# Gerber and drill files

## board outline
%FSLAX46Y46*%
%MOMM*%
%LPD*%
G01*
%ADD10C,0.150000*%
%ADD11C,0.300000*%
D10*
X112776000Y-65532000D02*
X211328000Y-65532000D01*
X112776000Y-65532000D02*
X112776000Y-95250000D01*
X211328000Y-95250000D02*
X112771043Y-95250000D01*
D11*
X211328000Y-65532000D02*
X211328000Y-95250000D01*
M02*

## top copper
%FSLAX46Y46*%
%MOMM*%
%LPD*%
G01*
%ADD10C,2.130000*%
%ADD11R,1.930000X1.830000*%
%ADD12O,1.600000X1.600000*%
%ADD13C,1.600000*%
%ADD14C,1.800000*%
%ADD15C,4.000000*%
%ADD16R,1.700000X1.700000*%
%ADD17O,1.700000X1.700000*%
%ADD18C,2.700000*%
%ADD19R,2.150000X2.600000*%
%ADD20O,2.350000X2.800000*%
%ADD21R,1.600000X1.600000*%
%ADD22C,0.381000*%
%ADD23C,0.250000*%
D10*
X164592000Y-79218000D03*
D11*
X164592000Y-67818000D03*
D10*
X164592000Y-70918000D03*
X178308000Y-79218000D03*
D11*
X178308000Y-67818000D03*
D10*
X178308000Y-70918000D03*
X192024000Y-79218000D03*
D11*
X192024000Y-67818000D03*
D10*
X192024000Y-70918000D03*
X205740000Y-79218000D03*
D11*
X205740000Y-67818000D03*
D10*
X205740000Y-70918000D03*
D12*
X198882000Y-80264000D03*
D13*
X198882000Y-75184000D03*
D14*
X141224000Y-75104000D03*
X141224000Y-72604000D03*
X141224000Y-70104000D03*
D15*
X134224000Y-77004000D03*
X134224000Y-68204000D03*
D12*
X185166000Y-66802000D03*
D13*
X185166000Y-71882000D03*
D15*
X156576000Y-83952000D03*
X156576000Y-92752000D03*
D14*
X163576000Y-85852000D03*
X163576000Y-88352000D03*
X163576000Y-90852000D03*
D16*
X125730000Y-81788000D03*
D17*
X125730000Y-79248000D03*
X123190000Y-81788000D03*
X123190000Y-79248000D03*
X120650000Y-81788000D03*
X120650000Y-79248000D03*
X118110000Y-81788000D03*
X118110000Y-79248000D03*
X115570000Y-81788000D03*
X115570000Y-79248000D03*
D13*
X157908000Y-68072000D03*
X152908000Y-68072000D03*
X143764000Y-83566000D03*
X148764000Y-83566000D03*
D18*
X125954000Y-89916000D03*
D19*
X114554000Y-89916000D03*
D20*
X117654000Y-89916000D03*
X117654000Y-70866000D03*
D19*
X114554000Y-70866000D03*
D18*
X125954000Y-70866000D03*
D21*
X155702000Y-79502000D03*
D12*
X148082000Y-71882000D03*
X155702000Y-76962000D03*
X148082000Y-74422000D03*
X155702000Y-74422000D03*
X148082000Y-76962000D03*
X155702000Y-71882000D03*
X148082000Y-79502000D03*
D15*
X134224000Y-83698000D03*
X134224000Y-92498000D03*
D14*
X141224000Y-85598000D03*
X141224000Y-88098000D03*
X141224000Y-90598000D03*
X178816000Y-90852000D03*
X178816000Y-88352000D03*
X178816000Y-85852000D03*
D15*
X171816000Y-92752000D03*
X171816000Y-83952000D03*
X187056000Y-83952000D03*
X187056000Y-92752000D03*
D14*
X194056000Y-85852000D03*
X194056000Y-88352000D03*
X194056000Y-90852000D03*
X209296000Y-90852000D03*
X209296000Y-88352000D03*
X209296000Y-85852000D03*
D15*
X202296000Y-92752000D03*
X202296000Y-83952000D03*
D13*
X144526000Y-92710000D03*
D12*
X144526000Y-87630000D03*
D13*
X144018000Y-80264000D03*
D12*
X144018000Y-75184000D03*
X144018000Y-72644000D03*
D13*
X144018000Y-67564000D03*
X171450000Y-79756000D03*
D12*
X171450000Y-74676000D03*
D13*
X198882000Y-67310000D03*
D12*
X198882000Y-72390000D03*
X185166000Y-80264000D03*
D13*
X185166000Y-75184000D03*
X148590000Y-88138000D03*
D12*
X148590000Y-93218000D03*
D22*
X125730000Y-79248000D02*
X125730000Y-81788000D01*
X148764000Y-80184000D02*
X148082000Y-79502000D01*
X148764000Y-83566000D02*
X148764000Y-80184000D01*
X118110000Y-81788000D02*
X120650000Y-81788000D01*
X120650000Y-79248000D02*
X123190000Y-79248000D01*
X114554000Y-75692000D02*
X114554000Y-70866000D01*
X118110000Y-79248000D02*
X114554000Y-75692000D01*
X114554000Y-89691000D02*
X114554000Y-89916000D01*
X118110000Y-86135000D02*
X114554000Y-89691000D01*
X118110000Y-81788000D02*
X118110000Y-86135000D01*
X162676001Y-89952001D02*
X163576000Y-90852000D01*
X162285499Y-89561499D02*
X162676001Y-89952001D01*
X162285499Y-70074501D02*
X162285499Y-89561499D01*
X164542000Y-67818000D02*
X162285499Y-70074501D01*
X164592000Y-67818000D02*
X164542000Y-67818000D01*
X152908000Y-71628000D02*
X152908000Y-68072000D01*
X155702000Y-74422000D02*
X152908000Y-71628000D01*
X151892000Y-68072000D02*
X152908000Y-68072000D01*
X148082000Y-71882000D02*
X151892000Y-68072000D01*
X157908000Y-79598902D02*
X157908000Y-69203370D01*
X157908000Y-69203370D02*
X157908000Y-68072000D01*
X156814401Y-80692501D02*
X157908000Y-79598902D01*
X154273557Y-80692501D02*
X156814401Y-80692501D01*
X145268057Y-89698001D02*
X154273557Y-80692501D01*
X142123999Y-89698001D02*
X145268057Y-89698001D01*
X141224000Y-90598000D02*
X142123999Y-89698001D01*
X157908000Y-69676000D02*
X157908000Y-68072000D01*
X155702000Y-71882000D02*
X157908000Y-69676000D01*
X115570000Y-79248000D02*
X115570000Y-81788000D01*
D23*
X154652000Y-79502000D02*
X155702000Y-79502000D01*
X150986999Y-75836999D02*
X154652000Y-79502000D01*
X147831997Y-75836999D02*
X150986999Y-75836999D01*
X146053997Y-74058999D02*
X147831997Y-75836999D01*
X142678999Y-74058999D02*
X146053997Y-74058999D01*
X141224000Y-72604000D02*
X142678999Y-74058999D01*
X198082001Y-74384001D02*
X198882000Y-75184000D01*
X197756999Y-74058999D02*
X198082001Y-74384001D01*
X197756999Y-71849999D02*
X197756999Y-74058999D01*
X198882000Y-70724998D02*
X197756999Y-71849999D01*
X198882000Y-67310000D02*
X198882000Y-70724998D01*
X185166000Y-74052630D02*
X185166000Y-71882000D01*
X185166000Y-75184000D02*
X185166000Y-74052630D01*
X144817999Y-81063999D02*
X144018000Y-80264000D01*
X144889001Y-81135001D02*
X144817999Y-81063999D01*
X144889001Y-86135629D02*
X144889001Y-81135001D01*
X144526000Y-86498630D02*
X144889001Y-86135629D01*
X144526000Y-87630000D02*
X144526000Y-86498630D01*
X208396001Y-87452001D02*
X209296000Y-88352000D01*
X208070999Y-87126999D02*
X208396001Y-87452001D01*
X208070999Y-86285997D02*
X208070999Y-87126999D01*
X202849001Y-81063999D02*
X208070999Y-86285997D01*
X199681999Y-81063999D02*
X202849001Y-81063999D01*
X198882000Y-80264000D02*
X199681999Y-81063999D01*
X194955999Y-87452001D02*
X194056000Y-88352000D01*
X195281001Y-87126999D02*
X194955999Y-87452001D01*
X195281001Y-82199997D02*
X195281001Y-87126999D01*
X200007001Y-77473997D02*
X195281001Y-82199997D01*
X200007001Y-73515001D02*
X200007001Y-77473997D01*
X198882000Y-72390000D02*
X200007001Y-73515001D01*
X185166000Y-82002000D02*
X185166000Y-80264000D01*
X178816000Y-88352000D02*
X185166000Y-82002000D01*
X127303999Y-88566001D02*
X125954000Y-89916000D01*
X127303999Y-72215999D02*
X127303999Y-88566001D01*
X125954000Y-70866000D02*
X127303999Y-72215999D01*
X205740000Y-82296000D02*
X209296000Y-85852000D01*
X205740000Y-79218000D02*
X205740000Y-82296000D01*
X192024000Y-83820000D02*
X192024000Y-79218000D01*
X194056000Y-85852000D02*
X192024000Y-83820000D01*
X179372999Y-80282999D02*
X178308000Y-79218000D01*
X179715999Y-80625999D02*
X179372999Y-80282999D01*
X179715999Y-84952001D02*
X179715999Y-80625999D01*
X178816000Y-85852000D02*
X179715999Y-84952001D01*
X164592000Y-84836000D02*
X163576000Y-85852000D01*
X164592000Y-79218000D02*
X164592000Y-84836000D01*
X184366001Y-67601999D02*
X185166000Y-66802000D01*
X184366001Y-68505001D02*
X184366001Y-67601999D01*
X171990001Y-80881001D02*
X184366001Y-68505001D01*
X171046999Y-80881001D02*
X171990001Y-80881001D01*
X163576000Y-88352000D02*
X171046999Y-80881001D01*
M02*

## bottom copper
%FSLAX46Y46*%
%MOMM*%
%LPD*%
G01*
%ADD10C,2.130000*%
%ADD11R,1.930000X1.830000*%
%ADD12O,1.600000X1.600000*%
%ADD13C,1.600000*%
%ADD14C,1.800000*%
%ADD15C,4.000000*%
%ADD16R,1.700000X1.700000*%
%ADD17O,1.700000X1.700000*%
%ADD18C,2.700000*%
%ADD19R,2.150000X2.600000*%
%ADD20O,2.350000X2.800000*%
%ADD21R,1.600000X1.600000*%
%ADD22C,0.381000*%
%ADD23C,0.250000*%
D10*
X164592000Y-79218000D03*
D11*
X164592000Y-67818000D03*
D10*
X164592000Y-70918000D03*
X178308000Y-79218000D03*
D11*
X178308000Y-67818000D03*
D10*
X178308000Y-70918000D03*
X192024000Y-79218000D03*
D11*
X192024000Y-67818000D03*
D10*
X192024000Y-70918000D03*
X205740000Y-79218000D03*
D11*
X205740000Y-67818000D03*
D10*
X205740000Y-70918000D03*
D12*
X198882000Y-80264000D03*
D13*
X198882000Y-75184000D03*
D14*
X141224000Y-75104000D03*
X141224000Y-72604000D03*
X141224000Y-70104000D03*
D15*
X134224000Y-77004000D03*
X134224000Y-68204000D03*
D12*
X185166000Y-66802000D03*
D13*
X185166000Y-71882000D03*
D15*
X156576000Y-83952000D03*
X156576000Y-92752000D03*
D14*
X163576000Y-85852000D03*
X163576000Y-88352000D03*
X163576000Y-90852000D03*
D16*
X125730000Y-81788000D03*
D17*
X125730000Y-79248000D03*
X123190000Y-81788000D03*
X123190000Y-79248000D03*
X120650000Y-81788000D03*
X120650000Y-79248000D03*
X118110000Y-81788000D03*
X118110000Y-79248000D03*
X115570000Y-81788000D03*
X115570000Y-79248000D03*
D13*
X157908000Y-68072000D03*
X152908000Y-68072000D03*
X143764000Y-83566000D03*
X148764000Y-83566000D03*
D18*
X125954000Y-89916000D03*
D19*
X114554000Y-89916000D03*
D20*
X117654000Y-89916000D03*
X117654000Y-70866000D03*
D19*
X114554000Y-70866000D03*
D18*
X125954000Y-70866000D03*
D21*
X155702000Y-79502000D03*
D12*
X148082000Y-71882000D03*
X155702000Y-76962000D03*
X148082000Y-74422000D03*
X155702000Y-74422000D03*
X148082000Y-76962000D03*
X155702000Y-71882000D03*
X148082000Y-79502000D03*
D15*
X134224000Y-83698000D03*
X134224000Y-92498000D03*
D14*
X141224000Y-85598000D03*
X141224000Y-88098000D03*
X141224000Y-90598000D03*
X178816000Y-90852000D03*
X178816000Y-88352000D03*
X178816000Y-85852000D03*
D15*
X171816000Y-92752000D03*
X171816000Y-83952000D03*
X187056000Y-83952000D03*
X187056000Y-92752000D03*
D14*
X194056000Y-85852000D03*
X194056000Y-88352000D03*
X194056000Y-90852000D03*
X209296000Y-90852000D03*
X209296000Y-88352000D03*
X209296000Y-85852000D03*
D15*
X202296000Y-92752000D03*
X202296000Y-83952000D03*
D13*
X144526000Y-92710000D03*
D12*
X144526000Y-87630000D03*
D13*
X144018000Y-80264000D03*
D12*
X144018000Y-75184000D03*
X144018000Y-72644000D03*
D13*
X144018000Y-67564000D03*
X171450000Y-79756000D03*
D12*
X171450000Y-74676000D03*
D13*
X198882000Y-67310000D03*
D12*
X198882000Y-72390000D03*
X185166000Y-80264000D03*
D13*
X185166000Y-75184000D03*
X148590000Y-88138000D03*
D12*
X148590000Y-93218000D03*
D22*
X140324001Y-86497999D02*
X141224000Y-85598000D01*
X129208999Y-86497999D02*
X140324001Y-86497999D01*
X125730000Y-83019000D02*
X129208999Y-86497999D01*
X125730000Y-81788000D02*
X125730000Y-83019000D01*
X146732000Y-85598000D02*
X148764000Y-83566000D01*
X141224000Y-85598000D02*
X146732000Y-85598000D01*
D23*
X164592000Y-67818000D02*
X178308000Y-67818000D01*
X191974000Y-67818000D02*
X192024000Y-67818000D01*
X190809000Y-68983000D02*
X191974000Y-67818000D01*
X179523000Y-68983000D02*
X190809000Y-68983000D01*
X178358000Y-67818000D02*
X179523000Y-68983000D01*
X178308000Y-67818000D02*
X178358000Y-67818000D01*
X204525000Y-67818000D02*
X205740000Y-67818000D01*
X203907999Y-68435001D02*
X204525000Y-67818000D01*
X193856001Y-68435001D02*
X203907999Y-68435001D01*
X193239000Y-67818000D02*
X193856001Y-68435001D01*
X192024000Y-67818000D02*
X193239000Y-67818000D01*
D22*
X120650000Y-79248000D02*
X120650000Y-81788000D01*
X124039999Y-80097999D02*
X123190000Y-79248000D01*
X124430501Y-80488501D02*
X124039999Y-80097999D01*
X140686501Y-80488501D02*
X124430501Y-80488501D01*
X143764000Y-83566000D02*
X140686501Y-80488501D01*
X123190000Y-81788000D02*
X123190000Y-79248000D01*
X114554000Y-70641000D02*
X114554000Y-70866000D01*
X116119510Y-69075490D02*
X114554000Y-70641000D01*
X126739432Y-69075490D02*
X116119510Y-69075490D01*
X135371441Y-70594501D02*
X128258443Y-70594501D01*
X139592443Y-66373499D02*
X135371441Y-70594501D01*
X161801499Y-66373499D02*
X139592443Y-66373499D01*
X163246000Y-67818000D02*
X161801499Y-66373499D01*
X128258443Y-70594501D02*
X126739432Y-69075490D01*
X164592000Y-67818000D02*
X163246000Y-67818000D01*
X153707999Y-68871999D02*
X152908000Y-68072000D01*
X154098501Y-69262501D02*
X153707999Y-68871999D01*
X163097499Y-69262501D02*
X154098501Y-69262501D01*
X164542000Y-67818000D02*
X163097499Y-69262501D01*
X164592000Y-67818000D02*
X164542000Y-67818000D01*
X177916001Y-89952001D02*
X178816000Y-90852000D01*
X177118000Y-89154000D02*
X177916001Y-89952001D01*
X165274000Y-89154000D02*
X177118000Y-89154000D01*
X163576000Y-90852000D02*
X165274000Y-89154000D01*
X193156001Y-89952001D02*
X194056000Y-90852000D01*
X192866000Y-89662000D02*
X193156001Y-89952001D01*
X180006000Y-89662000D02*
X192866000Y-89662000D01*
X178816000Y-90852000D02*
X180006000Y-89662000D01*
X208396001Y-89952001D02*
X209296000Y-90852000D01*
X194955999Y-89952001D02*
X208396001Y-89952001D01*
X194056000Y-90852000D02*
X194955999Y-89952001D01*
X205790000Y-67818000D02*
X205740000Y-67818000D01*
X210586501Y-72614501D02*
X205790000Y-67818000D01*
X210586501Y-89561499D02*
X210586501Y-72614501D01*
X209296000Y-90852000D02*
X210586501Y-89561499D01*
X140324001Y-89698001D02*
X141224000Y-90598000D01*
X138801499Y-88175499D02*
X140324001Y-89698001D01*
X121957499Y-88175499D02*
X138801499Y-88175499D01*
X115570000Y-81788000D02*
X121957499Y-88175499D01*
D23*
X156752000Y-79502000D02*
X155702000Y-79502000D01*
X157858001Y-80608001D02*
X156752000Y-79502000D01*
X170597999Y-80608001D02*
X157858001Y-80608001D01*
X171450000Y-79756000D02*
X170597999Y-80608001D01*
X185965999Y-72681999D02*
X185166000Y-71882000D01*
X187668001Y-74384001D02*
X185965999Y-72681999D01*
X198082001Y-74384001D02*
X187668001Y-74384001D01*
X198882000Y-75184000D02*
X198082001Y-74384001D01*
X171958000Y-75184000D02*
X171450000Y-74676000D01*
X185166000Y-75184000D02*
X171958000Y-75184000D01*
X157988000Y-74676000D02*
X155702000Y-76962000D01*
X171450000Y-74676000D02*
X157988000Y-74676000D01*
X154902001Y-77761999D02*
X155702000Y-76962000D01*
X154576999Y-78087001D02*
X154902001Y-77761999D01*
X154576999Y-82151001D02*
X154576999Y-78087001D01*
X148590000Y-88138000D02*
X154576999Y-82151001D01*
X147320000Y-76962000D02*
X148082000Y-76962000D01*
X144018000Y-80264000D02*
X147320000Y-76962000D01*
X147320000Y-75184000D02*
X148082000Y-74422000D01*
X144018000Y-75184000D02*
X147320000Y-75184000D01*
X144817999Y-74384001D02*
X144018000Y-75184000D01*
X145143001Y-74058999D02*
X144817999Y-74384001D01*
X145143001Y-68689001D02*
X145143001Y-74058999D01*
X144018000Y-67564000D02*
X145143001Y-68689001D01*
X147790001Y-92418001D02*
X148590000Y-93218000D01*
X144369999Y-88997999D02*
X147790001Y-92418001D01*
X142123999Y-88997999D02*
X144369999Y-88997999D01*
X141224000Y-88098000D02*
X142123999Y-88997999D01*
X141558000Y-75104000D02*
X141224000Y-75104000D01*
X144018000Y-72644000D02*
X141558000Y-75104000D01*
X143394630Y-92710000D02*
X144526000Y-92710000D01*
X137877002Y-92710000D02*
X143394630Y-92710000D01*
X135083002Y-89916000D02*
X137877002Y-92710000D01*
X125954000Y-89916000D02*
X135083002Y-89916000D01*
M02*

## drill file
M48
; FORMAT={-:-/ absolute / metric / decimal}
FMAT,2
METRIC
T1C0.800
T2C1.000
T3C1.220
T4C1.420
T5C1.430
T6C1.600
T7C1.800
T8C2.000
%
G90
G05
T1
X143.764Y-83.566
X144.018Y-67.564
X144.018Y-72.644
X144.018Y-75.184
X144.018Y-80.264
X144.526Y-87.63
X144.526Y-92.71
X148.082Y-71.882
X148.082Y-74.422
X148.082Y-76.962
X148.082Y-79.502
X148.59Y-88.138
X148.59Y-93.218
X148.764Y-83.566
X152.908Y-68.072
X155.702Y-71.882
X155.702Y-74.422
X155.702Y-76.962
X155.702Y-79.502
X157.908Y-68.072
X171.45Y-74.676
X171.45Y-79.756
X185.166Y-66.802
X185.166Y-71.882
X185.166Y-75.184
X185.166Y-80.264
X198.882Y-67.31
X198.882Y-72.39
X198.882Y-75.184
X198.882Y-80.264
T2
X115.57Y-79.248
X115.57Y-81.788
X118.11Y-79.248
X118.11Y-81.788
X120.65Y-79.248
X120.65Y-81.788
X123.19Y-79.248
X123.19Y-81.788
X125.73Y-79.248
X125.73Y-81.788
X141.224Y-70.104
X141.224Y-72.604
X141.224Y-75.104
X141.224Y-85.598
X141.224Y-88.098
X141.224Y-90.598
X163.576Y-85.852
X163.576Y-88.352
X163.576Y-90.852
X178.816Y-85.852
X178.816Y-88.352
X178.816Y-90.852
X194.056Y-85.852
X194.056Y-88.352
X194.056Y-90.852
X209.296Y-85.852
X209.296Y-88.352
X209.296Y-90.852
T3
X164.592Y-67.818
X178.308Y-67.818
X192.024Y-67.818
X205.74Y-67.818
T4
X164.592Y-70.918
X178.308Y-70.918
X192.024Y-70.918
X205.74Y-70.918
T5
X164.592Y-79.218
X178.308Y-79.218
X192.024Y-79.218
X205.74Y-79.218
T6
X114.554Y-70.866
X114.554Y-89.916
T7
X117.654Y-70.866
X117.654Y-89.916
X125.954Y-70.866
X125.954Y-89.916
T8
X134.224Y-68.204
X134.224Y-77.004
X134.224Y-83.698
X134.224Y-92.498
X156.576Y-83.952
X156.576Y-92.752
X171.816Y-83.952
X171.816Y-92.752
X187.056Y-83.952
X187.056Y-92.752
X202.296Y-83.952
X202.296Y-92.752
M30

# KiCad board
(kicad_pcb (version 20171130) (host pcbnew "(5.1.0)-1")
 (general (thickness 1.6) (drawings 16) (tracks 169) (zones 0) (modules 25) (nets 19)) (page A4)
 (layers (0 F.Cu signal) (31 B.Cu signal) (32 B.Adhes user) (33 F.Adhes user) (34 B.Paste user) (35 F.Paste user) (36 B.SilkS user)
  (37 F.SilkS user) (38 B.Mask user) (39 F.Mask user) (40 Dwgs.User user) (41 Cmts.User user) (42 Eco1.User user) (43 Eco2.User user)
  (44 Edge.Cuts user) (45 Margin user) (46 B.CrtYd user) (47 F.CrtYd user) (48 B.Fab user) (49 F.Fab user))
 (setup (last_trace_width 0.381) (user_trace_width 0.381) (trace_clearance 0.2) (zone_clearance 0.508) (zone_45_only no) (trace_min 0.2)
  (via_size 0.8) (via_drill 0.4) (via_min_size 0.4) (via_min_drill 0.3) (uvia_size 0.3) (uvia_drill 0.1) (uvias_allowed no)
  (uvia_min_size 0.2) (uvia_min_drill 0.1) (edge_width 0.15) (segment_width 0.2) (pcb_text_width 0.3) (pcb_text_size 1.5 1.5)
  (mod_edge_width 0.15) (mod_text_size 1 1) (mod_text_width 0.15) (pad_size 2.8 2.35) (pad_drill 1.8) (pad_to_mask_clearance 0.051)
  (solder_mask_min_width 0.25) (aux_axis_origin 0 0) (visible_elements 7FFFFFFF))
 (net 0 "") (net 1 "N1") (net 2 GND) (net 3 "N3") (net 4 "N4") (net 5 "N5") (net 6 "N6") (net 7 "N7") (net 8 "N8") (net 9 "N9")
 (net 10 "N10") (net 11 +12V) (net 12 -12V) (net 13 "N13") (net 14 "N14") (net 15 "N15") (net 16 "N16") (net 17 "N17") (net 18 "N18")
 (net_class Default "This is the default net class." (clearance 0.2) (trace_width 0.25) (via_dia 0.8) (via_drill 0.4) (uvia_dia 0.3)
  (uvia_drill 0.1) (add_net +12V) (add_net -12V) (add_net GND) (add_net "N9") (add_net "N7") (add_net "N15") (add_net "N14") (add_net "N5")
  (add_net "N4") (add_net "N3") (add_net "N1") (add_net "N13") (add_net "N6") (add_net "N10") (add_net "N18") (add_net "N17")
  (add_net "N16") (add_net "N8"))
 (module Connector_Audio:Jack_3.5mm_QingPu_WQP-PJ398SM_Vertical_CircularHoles (layer F.Cu) (at 164.592 67.818)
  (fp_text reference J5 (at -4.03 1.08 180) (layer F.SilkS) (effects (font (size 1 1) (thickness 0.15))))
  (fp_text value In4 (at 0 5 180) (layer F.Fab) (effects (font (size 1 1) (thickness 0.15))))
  (pad T thru_hole circle (at 0 11.4 180) (size 2.13 2.13) (drill 1.43) (layers *.Cu *.Mask) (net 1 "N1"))
  (pad S thru_hole rect (at 0 0 180) (size 1.93 1.83) (drill 1.22) (layers *.Cu *.Mask) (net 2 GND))
  (pad TN thru_hole circle (at 0 3.1 180) (size 2.13 2.13) (drill 1.42) (layers *.Cu *.Mask)))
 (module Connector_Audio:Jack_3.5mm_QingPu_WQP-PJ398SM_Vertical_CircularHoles (layer F.Cu) (at 178.308 67.818)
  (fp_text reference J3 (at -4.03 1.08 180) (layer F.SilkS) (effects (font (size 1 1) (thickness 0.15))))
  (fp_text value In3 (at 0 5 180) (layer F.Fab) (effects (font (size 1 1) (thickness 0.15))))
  (pad T thru_hole circle (at 0 11.4 180) (size 2.13 2.13) (drill 1.43) (layers *.Cu *.Mask) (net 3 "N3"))
  (pad S thru_hole rect (at 0 0 180) (size 1.93 1.83) (drill 1.22) (layers *.Cu *.Mask) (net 2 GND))
  (pad TN thru_hole circle (at 0 3.1 180) (size 2.13 2.13) (drill 1.42) (layers *.Cu *.Mask)))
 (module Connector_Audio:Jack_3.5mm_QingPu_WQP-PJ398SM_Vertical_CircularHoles (layer F.Cu) (at 192.024 67.818)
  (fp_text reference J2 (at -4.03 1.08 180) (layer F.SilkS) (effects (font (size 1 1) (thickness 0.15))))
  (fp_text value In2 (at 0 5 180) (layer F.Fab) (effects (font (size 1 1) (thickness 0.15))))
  (pad T thru_hole circle (at 0 11.4 180) (size 2.13 2.13) (drill 1.43) (layers *.Cu *.Mask) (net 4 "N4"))
  (pad S thru_hole rect (at 0 0 180) (size 1.93 1.83) (drill 1.22) (layers *.Cu *.Mask) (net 2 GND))
  (pad TN thru_hole circle (at 0 3.1 180) (size 2.13 2.13) (drill 1.42) (layers *.Cu *.Mask)))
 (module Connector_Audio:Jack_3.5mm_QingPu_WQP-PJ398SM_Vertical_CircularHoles (layer F.Cu) (at 205.74 67.818)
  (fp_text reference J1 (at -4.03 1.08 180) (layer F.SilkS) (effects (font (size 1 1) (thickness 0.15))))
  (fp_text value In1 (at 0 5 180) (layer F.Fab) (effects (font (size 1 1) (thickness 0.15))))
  (pad T thru_hole circle (at 0 11.4 180) (size 2.13 2.13) (drill 1.43) (layers *.Cu *.Mask) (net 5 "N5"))
  (pad S thru_hole rect (at 0 0 180) (size 1.93 1.83) (drill 1.22) (layers *.Cu *.Mask) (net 2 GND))
  (pad TN thru_hole circle (at 0 3.1 180) (size 2.13 2.13) (drill 1.42) (layers *.Cu *.Mask)))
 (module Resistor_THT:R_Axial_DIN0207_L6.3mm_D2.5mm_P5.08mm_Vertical (layer F.Cu) (at 198.882 75.184 270)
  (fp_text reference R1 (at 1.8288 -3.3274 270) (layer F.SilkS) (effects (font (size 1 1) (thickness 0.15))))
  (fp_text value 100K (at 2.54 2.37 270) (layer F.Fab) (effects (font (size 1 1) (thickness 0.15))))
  (pad 2 thru_hole oval (at 5.08 0 270) (size 1.6 1.6) (drill 0.8) (layers *.Cu *.Mask) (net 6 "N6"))
  (pad 1 thru_hole circle (at 0 0 270) (size 1.6 1.6) (drill 0.8) (layers *.Cu *.Mask) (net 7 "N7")))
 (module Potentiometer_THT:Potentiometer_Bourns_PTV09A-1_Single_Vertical (layer F.Cu) (at 141.224 70.104 180)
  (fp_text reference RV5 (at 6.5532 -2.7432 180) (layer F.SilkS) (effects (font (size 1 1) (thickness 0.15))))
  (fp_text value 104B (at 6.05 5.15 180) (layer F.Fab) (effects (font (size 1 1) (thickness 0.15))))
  (pad 3 thru_hole circle (at 0 -5 180) (size 1.8 1.8) (drill 1) (layers *.Cu *.Mask) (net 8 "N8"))
  (pad 2 thru_hole circle (at 0 -2.5 180) (size 1.8 1.8) (drill 1) (layers *.Cu *.Mask) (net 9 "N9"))
  (pad 1 thru_hole circle (at 0 0 180) (size 1.8 1.8) (drill 1) (layers *.Cu *.Mask))
  (pad "" np_thru_hole circle (at 7 -6.9 180) (size 4 4) (drill 2) (layers *.Cu *.Mask))
  (pad "" np_thru_hole circle (at 7 1.9 180) (size 4 4) (drill 2) (layers *.Cu *.Mask)))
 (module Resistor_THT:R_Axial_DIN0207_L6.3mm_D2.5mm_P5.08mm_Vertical (layer F.Cu) (at 185.166 71.882 90)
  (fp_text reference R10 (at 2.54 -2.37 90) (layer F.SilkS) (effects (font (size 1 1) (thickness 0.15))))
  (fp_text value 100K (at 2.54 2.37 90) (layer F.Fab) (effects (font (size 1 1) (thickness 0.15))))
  (pad 2 thru_hole oval (at 5.08 0 90) (size 1.6 1.6) (drill 0.8) (layers *.Cu *.Mask) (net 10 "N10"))
  (pad 1 thru_hole circle (at 0 0 90) (size 1.6 1.6) (drill 0.8) (layers *.Cu *.Mask) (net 7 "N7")))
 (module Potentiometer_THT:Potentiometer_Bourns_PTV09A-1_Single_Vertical (layer F.Cu) (at 163.576 85.852 180)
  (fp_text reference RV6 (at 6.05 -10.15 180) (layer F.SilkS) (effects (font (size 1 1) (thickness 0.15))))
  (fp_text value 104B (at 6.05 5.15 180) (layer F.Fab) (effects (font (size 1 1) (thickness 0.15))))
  (pad "" np_thru_hole circle (at 7 1.9 180) (size 4 4) (drill 2) (layers *.Cu *.Mask))
  (pad "" np_thru_hole circle (at 7 -6.9 180) (size 4 4) (drill 2) (layers *.Cu *.Mask))
  (pad 1 thru_hole circle (at 0 0 180) (size 1.8 1.8) (drill 1) (layers *.Cu *.Mask) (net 1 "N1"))
  (pad 2 thru_hole circle (at 0 -2.5 180) (size 1.8 1.8) (drill 1) (layers *.Cu *.Mask) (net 10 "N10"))
  (pad 3 thru_hole circle (at 0 -5 180) (size 1.8 1.8) (drill 1) (layers *.Cu *.Mask) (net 2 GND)))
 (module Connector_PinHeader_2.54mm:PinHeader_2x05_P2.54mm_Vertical (layer B.Cu) (at 125.73 81.788 90)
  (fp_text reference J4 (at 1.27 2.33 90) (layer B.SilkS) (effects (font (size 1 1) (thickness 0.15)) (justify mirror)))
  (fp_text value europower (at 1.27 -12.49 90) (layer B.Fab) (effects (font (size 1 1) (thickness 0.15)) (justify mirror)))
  (pad 1 thru_hole rect (at 0 0 90) (size 1.7 1.7) (drill 1) (layers *.Cu *.Mask) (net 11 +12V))
  (pad 2 thru_hole oval (at 2.54 0 90) (size 1.7 1.7) (drill 1) (layers *.Cu *.Mask) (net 11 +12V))
  (pad 3 thru_hole oval (at 0 -2.54 90) (size 1.7 1.7) (drill 1) (layers *.Cu *.Mask) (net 2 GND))
  (pad 4 thru_hole oval (at 2.54 -2.54 90) (size 1.7 1.7) (drill 1) (layers *.Cu *.Mask) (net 2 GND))
  (pad 5 thru_hole oval (at 0 -5.08 90) (size 1.7 1.7) (drill 1) (layers *.Cu *.Mask) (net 2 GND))
  (pad 6 thru_hole oval (at 2.54 -5.08 90) (size 1.7 1.7) (drill 1) (layers *.Cu *.Mask) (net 2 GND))
  (pad 7 thru_hole oval (at 0 -7.62 90) (size 1.7 1.7) (drill 1) (layers *.Cu *.Mask) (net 2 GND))
  (pad 8 thru_hole oval (at 2.54 -7.62 90) (size 1.7 1.7) (drill 1) (layers *.Cu *.Mask) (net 2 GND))
  (pad 9 thru_hole oval (at 0 -10.16 90) (size 1.7 1.7) (drill 1) (layers *.Cu *.Mask) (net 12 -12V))
  (pad 10 thru_hole oval (at 2.54 -10.16 90) (size 1.7 1.7) (drill 1) (layers *.Cu *.Mask) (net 12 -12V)))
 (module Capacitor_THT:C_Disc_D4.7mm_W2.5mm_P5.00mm (layer F.Cu) (at 152.908 68.072)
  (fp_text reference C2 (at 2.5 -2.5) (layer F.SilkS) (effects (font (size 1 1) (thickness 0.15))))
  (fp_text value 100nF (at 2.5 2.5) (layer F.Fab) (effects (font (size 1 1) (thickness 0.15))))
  (pad 2 thru_hole circle (at 5 0) (size 1.6 1.6) (drill 0.8) (layers *.Cu *.Mask) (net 12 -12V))
  (pad 1 thru_hole circle (at 0 0) (size 1.6 1.6) (drill 0.8) (layers *.Cu *.Mask) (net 2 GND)))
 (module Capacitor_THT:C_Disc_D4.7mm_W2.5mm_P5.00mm (layer F.Cu) (at 143.764 83.566)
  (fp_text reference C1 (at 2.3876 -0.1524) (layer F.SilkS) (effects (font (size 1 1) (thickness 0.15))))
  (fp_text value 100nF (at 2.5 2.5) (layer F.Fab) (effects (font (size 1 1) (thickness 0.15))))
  (pad 1 thru_hole circle (at 0 0) (size 1.6 1.6) (drill 0.8) (layers *.Cu *.Mask) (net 2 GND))
  (pad 2 thru_hole circle (at 5 0) (size 1.6 1.6) (drill 0.8) (layers *.Cu *.Mask) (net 11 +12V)))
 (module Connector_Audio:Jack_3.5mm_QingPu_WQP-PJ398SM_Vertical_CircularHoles (layer F.Cu) (at 114.554 89.916 90)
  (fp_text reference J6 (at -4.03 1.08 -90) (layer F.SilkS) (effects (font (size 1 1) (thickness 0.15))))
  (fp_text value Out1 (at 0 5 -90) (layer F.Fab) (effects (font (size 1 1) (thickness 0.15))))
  (pad T thru_hole circle (at 0 11.4 270) (size 2.7 2.7) (drill 1.8) (layers *.Cu *.Mask) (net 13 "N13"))
  (pad S thru_hole rect (at 0 0 270) (size 2.6 2.15) (drill 1.6) (layers *.Cu *.Mask) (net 2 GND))
  (pad TN thru_hole oval (at 0 3.1 270) (size 2.8 2.35) (drill 1.8) (layers *.Cu *.Mask)))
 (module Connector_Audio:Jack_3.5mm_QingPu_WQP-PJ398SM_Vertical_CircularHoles (layer F.Cu) (at 114.554 70.866 90)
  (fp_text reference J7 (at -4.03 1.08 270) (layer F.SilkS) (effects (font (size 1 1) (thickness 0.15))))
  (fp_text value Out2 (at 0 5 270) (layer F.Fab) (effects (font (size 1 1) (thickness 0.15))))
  (pad TN thru_hole oval (at 0 3.1 270) (size 2.8 2.35) (drill 1.8) (layers *.Cu *.Mask))
  (pad S thru_hole rect (at 0 0 270) (size 2.6 2.15) (drill 1.6) (layers *.Cu *.Mask) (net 2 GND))
  (pad T thru_hole circle (at 0 11.4 270) (size 2.7 2.7) (drill 1.8) (layers *.Cu *.Mask) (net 13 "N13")))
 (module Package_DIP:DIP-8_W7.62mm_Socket (layer F.Cu) (at 155.702 79.502 180)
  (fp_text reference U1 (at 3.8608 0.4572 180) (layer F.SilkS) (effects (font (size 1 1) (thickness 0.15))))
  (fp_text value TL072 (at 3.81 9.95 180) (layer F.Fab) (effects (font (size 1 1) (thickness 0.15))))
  (pad 1 thru_hole rect (at 0 0 180) (size 1.6 1.6) (drill 0.8) (layers *.Cu *.Mask) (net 9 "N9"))
  (pad 5 thru_hole oval (at 7.62 7.62 180) (size 1.6 1.6) (drill 0.8) (layers *.Cu *.Mask) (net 2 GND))
  (pad 2 thru_hole oval (at 0 2.54 180) (size 1.6 1.6) (drill 0.8) (layers *.Cu *.Mask) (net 7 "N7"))
  (pad 6 thru_hole oval (at 7.62 5.08 180) (size 1.6 1.6) (drill 0.8) (layers *.Cu *.Mask) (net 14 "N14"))
  (pad 3 thru_hole oval (at 0 5.08 180) (size 1.6 1.6) (drill 0.8) (layers *.Cu *.Mask) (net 2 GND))
  (pad 7 thru_hole oval (at 7.62 2.54 180) (size 1.6 1.6) (drill 0.8) (layers *.Cu *.Mask) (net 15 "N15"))
  (pad 4 thru_hole oval (at 0 7.62 180) (size 1.6 1.6) (drill 0.8) (layers *.Cu *.Mask) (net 12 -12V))
  (pad 8 thru_hole oval (at 7.62 0 180) (size 1.6 1.6) (drill 0.8) (layers *.Cu *.Mask) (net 11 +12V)))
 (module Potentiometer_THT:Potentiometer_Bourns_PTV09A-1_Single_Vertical (layer F.Cu) (at 141.224 85.598 180)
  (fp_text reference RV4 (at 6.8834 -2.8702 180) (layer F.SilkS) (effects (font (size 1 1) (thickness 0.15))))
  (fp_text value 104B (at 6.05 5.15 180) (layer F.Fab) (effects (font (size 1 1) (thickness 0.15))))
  (pad "" np_thru_hole circle (at 7 1.9 180) (size 4 4) (drill 2) (layers *.Cu *.Mask))
  (pad "" np_thru_hole circle (at 7 -6.9 180) (size 4 4) (drill 2) (layers *.Cu *.Mask))
  (pad 1 thru_hole circle (at 0 0 180) (size 1.8 1.8) (drill 1) (layers *.Cu *.Mask) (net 11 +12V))
  (pad 2 thru_hole circle (at 0 -2.5 180) (size 1.8 1.8) (drill 1) (layers *.Cu *.Mask) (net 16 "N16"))
  (pad 3 thru_hole circle (at 0 -5 180) (size 1.8 1.8) (drill 1) (layers *.Cu *.Mask) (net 12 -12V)))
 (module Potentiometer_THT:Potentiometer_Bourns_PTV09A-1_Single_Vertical (layer F.Cu) (at 178.816 85.852 180)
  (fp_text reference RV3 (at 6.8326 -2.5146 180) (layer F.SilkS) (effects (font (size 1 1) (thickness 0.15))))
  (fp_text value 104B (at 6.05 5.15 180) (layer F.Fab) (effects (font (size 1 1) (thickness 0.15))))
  (pad 3 thru_hole circle (at 0 -5 180) (size 1.8 1.8) (drill 1) (layers *.Cu *.Mask) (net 2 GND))
  (pad 2 thru_hole circle (at 0 -2.5 180) (size 1.8 1.8) (drill 1) (layers *.Cu *.Mask) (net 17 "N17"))
  (pad 1 thru_hole circle (at 0 0 180) (size 1.8 1.8) (drill 1) (layers *.Cu *.Mask) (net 3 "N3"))
  (pad "" np_thru_hole circle (at 7 -6.9 180) (size 4 4) (drill 2) (layers *.Cu *.Mask))
  (pad "" np_thru_hole circle (at 7 1.9 180) (size 4 4) (drill 2) (layers *.Cu *.Mask)))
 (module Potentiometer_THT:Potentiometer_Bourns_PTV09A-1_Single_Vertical (layer F.Cu) (at 194.056 85.852 180)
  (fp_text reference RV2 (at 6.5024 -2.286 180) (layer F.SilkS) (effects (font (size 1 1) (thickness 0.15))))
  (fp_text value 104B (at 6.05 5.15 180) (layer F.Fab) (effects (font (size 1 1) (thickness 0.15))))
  (pad "" np_thru_hole circle (at 7 1.9 180) (size 4 4) (drill 2) (layers *.Cu *.Mask))
  (pad "" np_thru_hole circle (at 7 -6.9 180) (size 4 4) (drill 2) (layers *.Cu *.Mask))
  (pad 1 thru_hole circle (at 0 0 180) (size 1.8 1.8) (drill 1) (layers *.Cu *.Mask) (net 4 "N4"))
  (pad 2 thru_hole circle (at 0 -2.5 180) (size 1.8 1.8) (drill 1) (layers *.Cu *.Mask) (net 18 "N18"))
  (pad 3 thru_hole circle (at 0 -5 180) (size 1.8 1.8) (drill 1) (layers *.Cu *.Mask) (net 2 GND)))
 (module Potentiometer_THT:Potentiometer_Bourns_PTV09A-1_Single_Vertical (layer F.Cu) (at 209.296 85.852 180)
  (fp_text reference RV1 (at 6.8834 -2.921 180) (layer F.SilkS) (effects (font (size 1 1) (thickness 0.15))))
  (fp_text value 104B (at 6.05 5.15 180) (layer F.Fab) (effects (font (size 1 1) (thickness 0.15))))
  (pad 3 thru_hole circle (at 0 -5 180) (size 1.8 1.8) (drill 1) (layers *.Cu *.Mask) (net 2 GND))
  (pad 2 thru_hole circle (at 0 -2.5 180) (size 1.8 1.8) (drill 1) (layers *.Cu *.Mask) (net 6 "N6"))
  (pad 1 thru_hole circle (at 0 0 180) (size 1.8 1.8) (drill 1) (layers *.Cu *.Mask) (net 5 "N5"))
  (pad "" np_thru_hole circle (at 7 -6.9 180) (size 4 4) (drill 2) (layers *.Cu *.Mask))
  (pad "" np_thru_hole circle (at 7 1.9 180) (size 4 4) (drill 2) (layers *.Cu *.Mask)))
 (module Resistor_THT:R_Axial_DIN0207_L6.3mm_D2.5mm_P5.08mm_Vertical (layer F.Cu) (at 144.526 92.71 90)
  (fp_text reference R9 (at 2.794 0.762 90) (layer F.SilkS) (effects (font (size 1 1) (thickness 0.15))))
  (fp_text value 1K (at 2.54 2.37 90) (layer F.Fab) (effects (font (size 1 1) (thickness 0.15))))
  (pad 1 thru_hole circle (at 0 0 90) (size 1.6 1.6) (drill 0.8) (layers *.Cu *.Mask) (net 13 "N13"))
  (pad 2 thru_hole oval (at 5.08 0 90) (size 1.6 1.6) (drill 0.8) (layers *.Cu *.Mask) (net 15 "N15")))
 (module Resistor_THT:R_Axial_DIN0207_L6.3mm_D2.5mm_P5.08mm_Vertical (layer F.Cu) (at 144.018 80.264 90)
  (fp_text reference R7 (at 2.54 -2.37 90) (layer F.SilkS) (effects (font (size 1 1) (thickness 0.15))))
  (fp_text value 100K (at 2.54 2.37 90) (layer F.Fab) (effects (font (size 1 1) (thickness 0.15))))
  (pad 1 thru_hole circle (at 0 0 90) (size 1.6 1.6) (drill 0.8) (layers *.Cu *.Mask) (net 15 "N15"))
  (pad 2 thru_hole oval (at 5.08 0 90) (size 1.6 1.6) (drill 0.8) (layers *.Cu *.Mask) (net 14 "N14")))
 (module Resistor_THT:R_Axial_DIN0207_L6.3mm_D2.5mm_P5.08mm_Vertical (layer F.Cu) (at 144.018 67.564 270)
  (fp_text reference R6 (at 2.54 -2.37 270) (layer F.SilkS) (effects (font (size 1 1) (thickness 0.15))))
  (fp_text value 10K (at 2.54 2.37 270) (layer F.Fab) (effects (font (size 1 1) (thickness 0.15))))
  (pad 2 thru_hole oval (at 5.08 0 270) (size 1.6 1.6) (drill 0.8) (layers *.Cu *.Mask) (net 8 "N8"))
  (pad 1 thru_hole circle (at 0 0 270) (size 1.6 1.6) (drill 0.8) (layers *.Cu *.Mask) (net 14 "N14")))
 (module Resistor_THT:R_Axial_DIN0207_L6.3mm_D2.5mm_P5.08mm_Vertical (layer F.Cu) (at 171.45 79.756 90)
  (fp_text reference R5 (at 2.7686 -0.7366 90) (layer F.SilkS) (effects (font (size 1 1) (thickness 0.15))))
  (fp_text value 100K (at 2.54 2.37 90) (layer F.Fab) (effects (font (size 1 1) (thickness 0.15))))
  (pad 1 thru_hole circle (at 0 0 90) (size 1.6 1.6) (drill 0.8) (layers *.Cu *.Mask) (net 9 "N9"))
  (pad 2 thru_hole oval (at 5.08 0 90) (size 1.6 1.6) (drill 0.8) (layers *.Cu *.Mask) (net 7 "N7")))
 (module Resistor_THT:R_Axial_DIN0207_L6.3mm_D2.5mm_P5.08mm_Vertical (layer F.Cu) (at 198.882 67.31 270)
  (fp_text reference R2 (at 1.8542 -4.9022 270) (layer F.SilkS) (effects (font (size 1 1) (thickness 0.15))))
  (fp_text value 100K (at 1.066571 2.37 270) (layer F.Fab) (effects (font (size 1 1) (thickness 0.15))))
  (pad 1 thru_hole circle (at 0 0 270) (size 1.6 1.6) (drill 0.8) (layers *.Cu *.Mask) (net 7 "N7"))
  (pad 2 thru_hole oval (at 5.08 0 270) (size 1.6 1.6) (drill 0.8) (layers *.Cu *.Mask) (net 18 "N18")))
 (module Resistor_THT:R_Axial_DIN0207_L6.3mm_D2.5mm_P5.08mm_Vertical (layer F.Cu) (at 185.166 75.184 270)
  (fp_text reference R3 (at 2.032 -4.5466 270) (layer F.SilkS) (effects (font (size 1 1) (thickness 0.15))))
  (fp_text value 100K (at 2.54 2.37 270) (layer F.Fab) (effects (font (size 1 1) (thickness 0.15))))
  (pad 2 thru_hole oval (at 5.08 0 270) (size 1.6 1.6) (drill 0.8) (layers *.Cu *.Mask) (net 17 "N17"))
  (pad 1 thru_hole circle (at 0 0 270) (size 1.6 1.6) (drill 0.8) (layers *.Cu *.Mask) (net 7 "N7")))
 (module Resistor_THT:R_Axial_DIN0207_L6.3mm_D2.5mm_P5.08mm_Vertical (layer F.Cu) (at 148.59 88.138 270)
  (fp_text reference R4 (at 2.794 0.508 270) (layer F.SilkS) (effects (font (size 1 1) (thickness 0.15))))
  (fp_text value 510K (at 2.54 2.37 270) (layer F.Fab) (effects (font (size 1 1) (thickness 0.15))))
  (pad 1 thru_hole circle (at 0 0 270) (size 1.6 1.6) (drill 0.8) (layers *.Cu *.Mask) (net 7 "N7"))
  (pad 2 thru_hole oval (at 5.08 0 270) (size 1.6 1.6) (drill 0.8) (layers *.Cu *.Mask) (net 16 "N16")))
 (gr_line (start 112.776 65.532) (end 211.328 65.532) (layer Edge.Cuts) (width 0.15))
 (gr_line (start 112.776 65.532) (end 112.776 95.25) (layer Edge.Cuts) (width 0.15))
 (gr_line (start 211.328 95.25) (end 112.771043 95.25) (layer Edge.Cuts) (width 0.15))
 (gr_line (start 211.328 65.532) (end 211.328 95.25) (layer Edge.Cuts) (width 0.3))
 (segment (start 140.324001 86.497999) (end 141.224 85.598) (width 0.381) (layer B.Cu) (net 11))
 (segment (start 129.208999 86.497999) (end 140.324001 86.497999) (width 0.381) (layer B.Cu) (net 11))
 (segment (start 125.73 83.019) (end 129.208999 86.497999) (width 0.381) (layer B.Cu) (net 11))
 (segment (start 125.73 81.788) (end 125.73 83.019) (width 0.381) (layer B.Cu) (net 11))
 (segment (start 146.732 85.598) (end 148.764 83.566) (width 0.381) (layer B.Cu) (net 11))
 (segment (start 141.224 85.598) (end 146.732 85.598) (width 0.381) (layer B.Cu) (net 11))
 (segment (start 125.73 79.248) (end 125.73 81.788) (width 0.381) (layer F.Cu) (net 11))
 (segment (start 148.764 80.184) (end 148.082 79.502) (width 0.381) (layer F.Cu) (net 11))
 (segment (start 148.764 83.566) (end 148.764 80.184) (width 0.381) (layer F.Cu) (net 11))
 (segment (start 164.592 67.818) (end 178.308 67.818) (width 0.25) (layer B.Cu) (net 2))
 (segment (start 191.974 67.818) (end 192.024 67.818) (width 0.25) (layer B.Cu) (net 2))
 (segment (start 190.809 68.983) (end 191.974 67.818) (width 0.25) (layer B.Cu) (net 2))
 (segment (start 179.523 68.983) (end 190.809 68.983) (width 0.25) (layer B.Cu) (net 2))
 (segment (start 178.358 67.818) (end 179.523 68.983) (width 0.25) (layer B.Cu) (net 2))
 (segment (start 178.308 67.818) (end 178.358 67.818) (width 0.25) (layer B.Cu) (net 2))
 (segment (start 204.525 67.818) (end 205.74 67.818) (width 0.25) (layer B.Cu) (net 2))
 (segment (start 203.907999 68.435001) (end 204.525 67.818) (width 0.25) (layer B.Cu) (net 2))
 (segment (start 193.856001 68.435001) (end 203.907999 68.435001) (width 0.25) (layer B.Cu) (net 2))
 (segment (start 193.239 67.818) (end 193.856001 68.435001) (width 0.25) (layer B.Cu) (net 2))
 (segment (start 192.024 67.818) (end 193.239 67.818) (width 0.25) (layer B.Cu) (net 2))
 (segment (start 120.65 79.248) (end 120.65 81.788) (width 0.381) (layer B.Cu) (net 2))
 (segment (start 118.11 81.788) (end 120.65 81.788) (width 0.381) (layer F.Cu) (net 2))
 (segment (start 120.65 79.248) (end 123.19 79.248) (width 0.381) (layer F.Cu) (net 2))
 (segment (start 114.554 75.692) (end 114.554 70.866) (width 0.381) (layer F.Cu) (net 2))
 (segment (start 118.11 79.248) (end 114.554 75.692) (width 0.381) (layer F.Cu) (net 2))
 (segment (start 124.039999 80.097999) (end 123.19 79.248) (width 0.381) (layer B.Cu) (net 2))
 (segment (start 124.430501 80.488501) (end 124.039999 80.097999) (width 0.381) (layer B.Cu) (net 2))
 (segment (start 140.686501 80.488501) (end 124.430501 80.488501) (width 0.381) (layer B.Cu) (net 2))
 (segment (start 143.764 83.566) (end 140.686501 80.488501) (width 0.381) (layer B.Cu) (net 2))
 (segment (start 123.19 81.788) (end 123.19 79.248) (width 0.381) (layer B.Cu) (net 2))
 (segment (start 114.554 89.691) (end 114.554 89.916) (width 0.381) (layer F.Cu) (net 2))
 (segment (start 118.11 86.135) (end 114.554 89.691) (width 0.381) (layer F.Cu) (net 2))
 (segment (start 118.11 81.788) (end 118.11 86.135) (width 0.381) (layer F.Cu) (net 2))
 (segment (start 114.554 70.641) (end 114.554 70.866) (width 0.381) (layer B.Cu) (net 2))
 (segment (start 116.11951 69.07549) (end 114.554 70.641) (width 0.381) (layer B.Cu) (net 2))
 (segment (start 126.739432 69.07549) (end 116.11951 69.07549) (width 0.381) (layer B.Cu) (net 2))
 (segment (start 135.371441 70.594501) (end 128.258443 70.594501) (width 0.381) (layer B.Cu) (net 2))
 (segment (start 139.592443 66.373499) (end 135.371441 70.594501) (width 0.381) (layer B.Cu) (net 2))
 (segment (start 161.801499 66.373499) (end 139.592443 66.373499) (width 0.381) (layer B.Cu) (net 2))
 (segment (start 163.246 67.818) (end 161.801499 66.373499) (width 0.381) (layer B.Cu) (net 2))
 (segment (start 128.258443 70.594501) (end 126.739432 69.07549) (width 0.381) (layer B.Cu) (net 2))
 (segment (start 164.592 67.818) (end 163.246 67.818) (width 0.381) (layer B.Cu) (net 2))
 (segment (start 153.707999 68.871999) (end 152.908 68.072) (width 0.381) (layer B.Cu) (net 2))
 (segment (start 154.098501 69.262501) (end 153.707999 68.871999) (width 0.381) (layer B.Cu) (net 2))
 (segment (start 163.097499 69.262501) (end 154.098501 69.262501) (width 0.381) (layer B.Cu) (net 2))
 (segment (start 164.542 67.818) (end 163.097499 69.262501) (width 0.381) (layer B.Cu) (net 2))
 (segment (start 164.592 67.818) (end 164.542 67.818) (width 0.381) (layer B.Cu) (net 2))
 (segment (start 162.676001 89.952001) (end 163.576 90.852) (width 0.381) (layer F.Cu) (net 2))
 (segment (start 162.285499 89.561499) (end 162.676001 89.952001) (width 0.381) (layer F.Cu) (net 2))
 (segment (start 162.285499 70.074501) (end 162.285499 89.561499) (width 0.381) (layer F.Cu) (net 2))
 (segment (start 164.542 67.818) (end 162.285499 70.074501) (width 0.381) (layer F.Cu) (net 2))
 (segment (start 164.592 67.818) (end 164.542 67.818) (width 0.381) (layer F.Cu) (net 2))
 (segment (start 177.916001 89.952001) (end 178.816 90.852) (width 0.381) (layer B.Cu) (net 2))
 (segment (start 177.118 89.154) (end 177.916001 89.952001) (width 0.381) (layer B.Cu) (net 2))
 (segment (start 165.274 89.154) (end 177.118 89.154) (width 0.381) (layer B.Cu) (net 2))
 (segment (start 163.576 90.852) (end 165.274 89.154) (width 0.381) (layer B.Cu) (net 2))
 (segment (start 193.156001 89.952001) (end 194.056 90.852) (width 0.381) (layer B.Cu) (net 2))
 (segment (start 192.866 89.662) (end 193.156001 89.952001) (width 0.381) (layer B.Cu) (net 2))
 (segment (start 180.006 89.662) (end 192.866 89.662) (width 0.381) (layer B.Cu) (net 2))
 (segment (start 178.816 90.852) (end 180.006 89.662) (width 0.381) (layer B.Cu) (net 2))
 (segment (start 208.396001 89.952001) (end 209.296 90.852) (width 0.381) (layer B.Cu) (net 2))
 (segment (start 194.955999 89.952001) (end 208.396001 89.952001) (width 0.381) (layer B.Cu) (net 2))
 (segment (start 194.056 90.852) (end 194.955999 89.952001) (width 0.381) (layer B.Cu) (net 2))
 (segment (start 205.79 67.818) (end 205.74 67.818) (width 0.381) (layer B.Cu) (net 2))
 (segment (start 210.586501 72.614501) (end 205.79 67.818) (width 0.381) (layer B.Cu) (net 2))
 (segment (start 210.586501 89.561499) (end 210.586501 72.614501) (width 0.381) (layer B.Cu) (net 2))
 (segment (start 209.296 90.852) (end 210.586501 89.561499) (width 0.381) (layer B.Cu) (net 2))
 (segment (start 152.908 71.628) (end 152.908 68.072) (width 0.381) (layer F.Cu) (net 2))
 (segment (start 155.702 74.422) (end 152.908 71.628) (width 0.381) (layer F.Cu) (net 2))
 (segment (start 151.892 68.072) (end 152.908 68.072) (width 0.381) (layer F.Cu) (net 2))
 (segment (start 148.082 71.882) (end 151.892 68.072) (width 0.381) (layer F.Cu) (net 2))
 (segment (start 140.324001 89.698001) (end 141.224 90.598) (width 0.381) (layer B.Cu) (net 12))
 (segment (start 138.801499 88.175499) (end 140.324001 89.698001) (width 0.381) (layer B.Cu) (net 12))
 (segment (start 121.957499 88.175499) (end 138.801499 88.175499) (width 0.381) (layer B.Cu) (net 12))
 (segment (start 115.57 81.788) (end 121.957499 88.175499) (width 0.381) (layer B.Cu) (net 12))
 (segment (start 157.908 79.598902) (end 157.908 69.20337) (width 0.381) (layer F.Cu) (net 12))
 (segment (start 157.908 69.20337) (end 157.908 68.072) (width 0.381) (layer F.Cu) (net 12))
 (segment (start 156.814401 80.692501) (end 157.908 79.598902) (width 0.381) (layer F.Cu) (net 12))
 (segment (start 154.273557 80.692501) (end 156.814401 80.692501) (width 0.381) (layer F.Cu) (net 12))
 (segment (start 145.268057 89.698001) (end 154.273557 80.692501) (width 0.381) (layer F.Cu) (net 12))
 (segment (start 142.123999 89.698001) (end 145.268057 89.698001) (width 0.381) (layer F.Cu) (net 12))
 (segment (start 141.224 90.598) (end 142.123999 89.698001) (width 0.381) (layer F.Cu) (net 12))
 (segment (start 157.908 69.676) (end 157.908 68.072) (width 0.381) (layer F.Cu) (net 12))
 (segment (start 155.702 71.882) (end 157.908 69.676) (width 0.381) (layer F.Cu) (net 12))
 (segment (start 115.57 79.248) (end 115.57 81.788) (width 0.381) (layer F.Cu) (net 12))
 (segment (start 156.752 79.502) (end 155.702 79.502) (width 0.25) (layer B.Cu) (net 9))
 (segment (start 157.858001 80.608001) (end 156.752 79.502) (width 0.25) (layer B.Cu) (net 9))
 (segment (start 170.597999 80.608001) (end 157.858001 80.608001) (width 0.25) (layer B.Cu) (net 9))
 (segment (start 171.45 79.756) (end 170.597999 80.608001) (width 0.25) (layer B.Cu) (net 9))
 (segment (start 154.652 79.502) (end 155.702 79.502) (width 0.25) (layer F.Cu) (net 9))
 (segment (start 150.986999 75.836999) (end 154.652 79.502) (width 0.25) (layer F.Cu) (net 9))
 (segment (start 147.831997 75.836999) (end 150.986999 75.836999) (width 0.25) (layer F.Cu) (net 9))
 (segment (start 146.053997 74.058999) (end 147.831997 75.836999) (width 0.25) (layer F.Cu) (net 9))
 (segment (start 142.678999 74.058999) (end 146.053997 74.058999) (width 0.25) (layer F.Cu) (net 9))
 (segment (start 141.224 72.604) (end 142.678999 74.058999) (width 0.25) (layer F.Cu) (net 9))
 (segment (start 198.082001 74.384001) (end 198.882 75.184) (width 0.25) (layer F.Cu) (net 7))
 (segment (start 197.756999 74.058999) (end 198.082001 74.384001) (width 0.25) (layer F.Cu) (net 7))
 (segment (start 197.756999 71.849999) (end 197.756999 74.058999) (width 0.25) (layer F.Cu) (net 7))
 (segment (start 198.882 70.724998) (end 197.756999 71.849999) (width 0.25) (layer F.Cu) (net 7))
 (segment (start 198.882 67.31) (end 198.882 70.724998) (width 0.25) (layer F.Cu) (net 7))
 (segment (start 185.965999 72.681999) (end 185.166 71.882) (width 0.25) (layer B.Cu) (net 7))
 (segment (start 187.668001 74.384001) (end 185.965999 72.681999) (width 0.25) (layer B.Cu) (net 7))
 (segment (start 198.082001 74.384001) (end 187.668001 74.384001) (width 0.25) (layer B.Cu) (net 7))
 (segment (start 198.882 75.184) (end 198.082001 74.384001) (width 0.25) (layer B.Cu) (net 7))
 (segment (start 185.166 74.05263) (end 185.166 71.882) (width 0.25) (layer F.Cu) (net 7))
 (segment (start 185.166 75.184) (end 185.166 74.05263) (width 0.25) (layer F.Cu) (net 7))
 (segment (start 171.958 75.184) (end 171.45 74.676) (width 0.25) (layer B.Cu) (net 7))
 (segment (start 185.166 75.184) (end 171.958 75.184) (width 0.25) (layer B.Cu) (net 7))
 (segment (start 157.988 74.676) (end 155.702 76.962) (width 0.25) (layer B.Cu) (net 7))
 (segment (start 171.45 74.676) (end 157.988 74.676) (width 0.25) (layer B.Cu) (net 7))
 (segment (start 154.902001 77.761999) (end 155.702 76.962) (width 0.25) (layer B.Cu) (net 7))
 (segment (start 154.576999 78.087001) (end 154.902001 77.761999) (width 0.25) (layer B.Cu) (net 7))
 (segment (start 154.576999 82.151001) (end 154.576999 78.087001) (width 0.25) (layer B.Cu) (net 7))
 (segment (start 148.59 88.138) (end 154.576999 82.151001) (width 0.25) (layer B.Cu) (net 7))
 (segment (start 147.32 76.962) (end 148.082 76.962) (width 0.25) (layer B.Cu) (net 15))
 (segment (start 144.018 80.264) (end 147.32 76.962) (width 0.25) (layer B.Cu) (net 15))
 (segment (start 144.817999 81.063999) (end 144.018 80.264) (width 0.25) (layer F.Cu) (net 15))
 (segment (start 144.889001 81.135001) (end 144.817999 81.063999) (width 0.25) (layer F.Cu) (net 15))
 (segment (start 144.889001 86.135629) (end 144.889001 81.135001) (width 0.25) (layer F.Cu) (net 15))
 (segment (start 144.526 86.49863) (end 144.889001 86.135629) (width 0.25) (layer F.Cu) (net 15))
 (segment (start 144.526 87.63) (end 144.526 86.49863) (width 0.25) (layer F.Cu) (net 15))
 (segment (start 147.32 75.184) (end 148.082 74.422) (width 0.25) (layer B.Cu) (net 14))
 (segment (start 144.018 75.184) (end 147.32 75.184) (width 0.25) (layer B.Cu) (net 14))
 (segment (start 144.817999 74.384001) (end 144.018 75.184) (width 0.25) (layer B.Cu) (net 14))
 (segment (start 145.143001 74.058999) (end 144.817999 74.384001) (width 0.25) (layer B.Cu) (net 14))
 (segment (start 145.143001 68.689001) (end 145.143001 74.058999) (width 0.25) (layer B.Cu) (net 14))
 (segment (start 144.018 67.564) (end 145.143001 68.689001) (width 0.25) (layer B.Cu) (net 14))
 (segment (start 208.396001 87.452001) (end 209.296 88.352) (width 0.25) (layer F.Cu) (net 6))
 (segment (start 208.070999 87.126999) (end 208.396001 87.452001) (width 0.25) (layer F.Cu) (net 6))
 (segment (start 208.070999 86.285997) (end 208.070999 87.126999) (width 0.25) (layer F.Cu) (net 6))
 (segment (start 202.849001 81.063999) (end 208.070999 86.285997) (width 0.25) (layer F.Cu) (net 6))
 (segment (start 199.681999 81.063999) (end 202.849001 81.063999) (width 0.25) (layer F.Cu) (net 6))
 (segment (start 198.882 80.264) (end 199.681999 81.063999) (width 0.25) (layer F.Cu) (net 6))
 (segment (start 194.955999 87.452001) (end 194.056 88.352) (width 0.25) (layer F.Cu) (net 18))
 (segment (start 195.281001 87.126999) (end 194.955999 87.452001) (width 0.25) (layer F.Cu) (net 18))
 (segment (start 195.281001 82.199997) (end 195.281001 87.126999) (width 0.25) (layer F.Cu) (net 18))
 (segment (start 200.007001 77.473997) (end 195.281001 82.199997) (width 0.25) (layer F.Cu) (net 18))
 (segment (start 200.007001 73.515001) (end 200.007001 77.473997) (width 0.25) (layer F.Cu) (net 18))
 (segment (start 198.882 72.39) (end 200.007001 73.515001) (width 0.25) (layer F.Cu) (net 18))
 (segment (start 185.166 82.002) (end 185.166 80.264) (width 0.25) (layer F.Cu) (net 17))
 (segment (start 178.816 88.352) (end 185.166 82.002) (width 0.25) (layer F.Cu) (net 17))
 (segment (start 147.790001 92.418001) (end 148.59 93.218) (width 0.25) (layer B.Cu) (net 16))
 (segment (start 144.369999 88.997999) (end 147.790001 92.418001) (width 0.25) (layer B.Cu) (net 16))
 (segment (start 142.123999 88.997999) (end 144.369999 88.997999) (width 0.25) (layer B.Cu) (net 16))
 (segment (start 141.224 88.098) (end 142.123999 88.997999) (width 0.25) (layer B.Cu) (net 16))
 (segment (start 141.558 75.104) (end 141.224 75.104) (width 0.25) (layer B.Cu) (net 8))
 (segment (start 144.018 72.644) (end 141.558 75.104) (width 0.25) (layer B.Cu) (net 8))
 (segment (start 143.39463 92.71) (end 144.526 92.71) (width 0.25) (layer B.Cu) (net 13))
 (segment (start 137.877002 92.71) (end 143.39463 92.71) (width 0.25) (layer B.Cu) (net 13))
 (segment (start 135.083002 89.916) (end 137.877002 92.71) (width 0.25) (layer B.Cu) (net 13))
 (segment (start 125.954 89.916) (end 135.083002 89.916) (width 0.25) (layer B.Cu) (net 13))
 (segment (start 127.303999 88.566001) (end 125.954 89.916) (width 0.25) (layer F.Cu) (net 13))
 (segment (start 127.303999 72.215999) (end 127.303999 88.566001) (width 0.25) (layer F.Cu) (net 13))
 (segment (start 125.954 70.866) (end 127.303999 72.215999) (width 0.25) (layer F.Cu) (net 13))
 (segment (start 205.74 82.296) (end 209.296 85.852) (width 0.25) (layer F.Cu) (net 5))
 (segment (start 205.74 79.218) (end 205.74 82.296) (width 0.25) (layer F.Cu) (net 5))
 (segment (start 192.024 83.82) (end 192.024 79.218) (width 0.25) (layer F.Cu) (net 4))
 (segment (start 194.056 85.852) (end 192.024 83.82) (width 0.25) (layer F.Cu) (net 4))
 (segment (start 179.372999 80.282999) (end 178.308 79.218) (width 0.25) (layer F.Cu) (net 3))
 (segment (start 179.715999 80.625999) (end 179.372999 80.282999) (width 0.25) (layer F.Cu) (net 3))
 (segment (start 179.715999 84.952001) (end 179.715999 80.625999) (width 0.25) (layer F.Cu) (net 3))
 (segment (start 178.816 85.852) (end 179.715999 84.952001) (width 0.25) (layer F.Cu) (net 3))
 (segment (start 164.592 84.836) (end 163.576 85.852) (width 0.25) (layer F.Cu) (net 1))
 (segment (start 164.592 79.218) (end 164.592 84.836) (width 0.25) (layer F.Cu) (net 1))
 (segment (start 184.366001 67.601999) (end 185.166 66.802) (width 0.25) (layer F.Cu) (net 10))
 (segment (start 184.366001 68.505001) (end 184.366001 67.601999) (width 0.25) (layer F.Cu) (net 10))
 (segment (start 171.990001 80.881001) (end 184.366001 68.505001) (width 0.25) (layer F.Cu) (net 10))
 (segment (start 171.046999 80.881001) (end 171.990001 80.881001) (width 0.25) (layer F.Cu) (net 10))
 (segment (start 163.576 88.352) (end 171.046999 80.881001) (width 0.25) (layer F.Cu) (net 10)))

